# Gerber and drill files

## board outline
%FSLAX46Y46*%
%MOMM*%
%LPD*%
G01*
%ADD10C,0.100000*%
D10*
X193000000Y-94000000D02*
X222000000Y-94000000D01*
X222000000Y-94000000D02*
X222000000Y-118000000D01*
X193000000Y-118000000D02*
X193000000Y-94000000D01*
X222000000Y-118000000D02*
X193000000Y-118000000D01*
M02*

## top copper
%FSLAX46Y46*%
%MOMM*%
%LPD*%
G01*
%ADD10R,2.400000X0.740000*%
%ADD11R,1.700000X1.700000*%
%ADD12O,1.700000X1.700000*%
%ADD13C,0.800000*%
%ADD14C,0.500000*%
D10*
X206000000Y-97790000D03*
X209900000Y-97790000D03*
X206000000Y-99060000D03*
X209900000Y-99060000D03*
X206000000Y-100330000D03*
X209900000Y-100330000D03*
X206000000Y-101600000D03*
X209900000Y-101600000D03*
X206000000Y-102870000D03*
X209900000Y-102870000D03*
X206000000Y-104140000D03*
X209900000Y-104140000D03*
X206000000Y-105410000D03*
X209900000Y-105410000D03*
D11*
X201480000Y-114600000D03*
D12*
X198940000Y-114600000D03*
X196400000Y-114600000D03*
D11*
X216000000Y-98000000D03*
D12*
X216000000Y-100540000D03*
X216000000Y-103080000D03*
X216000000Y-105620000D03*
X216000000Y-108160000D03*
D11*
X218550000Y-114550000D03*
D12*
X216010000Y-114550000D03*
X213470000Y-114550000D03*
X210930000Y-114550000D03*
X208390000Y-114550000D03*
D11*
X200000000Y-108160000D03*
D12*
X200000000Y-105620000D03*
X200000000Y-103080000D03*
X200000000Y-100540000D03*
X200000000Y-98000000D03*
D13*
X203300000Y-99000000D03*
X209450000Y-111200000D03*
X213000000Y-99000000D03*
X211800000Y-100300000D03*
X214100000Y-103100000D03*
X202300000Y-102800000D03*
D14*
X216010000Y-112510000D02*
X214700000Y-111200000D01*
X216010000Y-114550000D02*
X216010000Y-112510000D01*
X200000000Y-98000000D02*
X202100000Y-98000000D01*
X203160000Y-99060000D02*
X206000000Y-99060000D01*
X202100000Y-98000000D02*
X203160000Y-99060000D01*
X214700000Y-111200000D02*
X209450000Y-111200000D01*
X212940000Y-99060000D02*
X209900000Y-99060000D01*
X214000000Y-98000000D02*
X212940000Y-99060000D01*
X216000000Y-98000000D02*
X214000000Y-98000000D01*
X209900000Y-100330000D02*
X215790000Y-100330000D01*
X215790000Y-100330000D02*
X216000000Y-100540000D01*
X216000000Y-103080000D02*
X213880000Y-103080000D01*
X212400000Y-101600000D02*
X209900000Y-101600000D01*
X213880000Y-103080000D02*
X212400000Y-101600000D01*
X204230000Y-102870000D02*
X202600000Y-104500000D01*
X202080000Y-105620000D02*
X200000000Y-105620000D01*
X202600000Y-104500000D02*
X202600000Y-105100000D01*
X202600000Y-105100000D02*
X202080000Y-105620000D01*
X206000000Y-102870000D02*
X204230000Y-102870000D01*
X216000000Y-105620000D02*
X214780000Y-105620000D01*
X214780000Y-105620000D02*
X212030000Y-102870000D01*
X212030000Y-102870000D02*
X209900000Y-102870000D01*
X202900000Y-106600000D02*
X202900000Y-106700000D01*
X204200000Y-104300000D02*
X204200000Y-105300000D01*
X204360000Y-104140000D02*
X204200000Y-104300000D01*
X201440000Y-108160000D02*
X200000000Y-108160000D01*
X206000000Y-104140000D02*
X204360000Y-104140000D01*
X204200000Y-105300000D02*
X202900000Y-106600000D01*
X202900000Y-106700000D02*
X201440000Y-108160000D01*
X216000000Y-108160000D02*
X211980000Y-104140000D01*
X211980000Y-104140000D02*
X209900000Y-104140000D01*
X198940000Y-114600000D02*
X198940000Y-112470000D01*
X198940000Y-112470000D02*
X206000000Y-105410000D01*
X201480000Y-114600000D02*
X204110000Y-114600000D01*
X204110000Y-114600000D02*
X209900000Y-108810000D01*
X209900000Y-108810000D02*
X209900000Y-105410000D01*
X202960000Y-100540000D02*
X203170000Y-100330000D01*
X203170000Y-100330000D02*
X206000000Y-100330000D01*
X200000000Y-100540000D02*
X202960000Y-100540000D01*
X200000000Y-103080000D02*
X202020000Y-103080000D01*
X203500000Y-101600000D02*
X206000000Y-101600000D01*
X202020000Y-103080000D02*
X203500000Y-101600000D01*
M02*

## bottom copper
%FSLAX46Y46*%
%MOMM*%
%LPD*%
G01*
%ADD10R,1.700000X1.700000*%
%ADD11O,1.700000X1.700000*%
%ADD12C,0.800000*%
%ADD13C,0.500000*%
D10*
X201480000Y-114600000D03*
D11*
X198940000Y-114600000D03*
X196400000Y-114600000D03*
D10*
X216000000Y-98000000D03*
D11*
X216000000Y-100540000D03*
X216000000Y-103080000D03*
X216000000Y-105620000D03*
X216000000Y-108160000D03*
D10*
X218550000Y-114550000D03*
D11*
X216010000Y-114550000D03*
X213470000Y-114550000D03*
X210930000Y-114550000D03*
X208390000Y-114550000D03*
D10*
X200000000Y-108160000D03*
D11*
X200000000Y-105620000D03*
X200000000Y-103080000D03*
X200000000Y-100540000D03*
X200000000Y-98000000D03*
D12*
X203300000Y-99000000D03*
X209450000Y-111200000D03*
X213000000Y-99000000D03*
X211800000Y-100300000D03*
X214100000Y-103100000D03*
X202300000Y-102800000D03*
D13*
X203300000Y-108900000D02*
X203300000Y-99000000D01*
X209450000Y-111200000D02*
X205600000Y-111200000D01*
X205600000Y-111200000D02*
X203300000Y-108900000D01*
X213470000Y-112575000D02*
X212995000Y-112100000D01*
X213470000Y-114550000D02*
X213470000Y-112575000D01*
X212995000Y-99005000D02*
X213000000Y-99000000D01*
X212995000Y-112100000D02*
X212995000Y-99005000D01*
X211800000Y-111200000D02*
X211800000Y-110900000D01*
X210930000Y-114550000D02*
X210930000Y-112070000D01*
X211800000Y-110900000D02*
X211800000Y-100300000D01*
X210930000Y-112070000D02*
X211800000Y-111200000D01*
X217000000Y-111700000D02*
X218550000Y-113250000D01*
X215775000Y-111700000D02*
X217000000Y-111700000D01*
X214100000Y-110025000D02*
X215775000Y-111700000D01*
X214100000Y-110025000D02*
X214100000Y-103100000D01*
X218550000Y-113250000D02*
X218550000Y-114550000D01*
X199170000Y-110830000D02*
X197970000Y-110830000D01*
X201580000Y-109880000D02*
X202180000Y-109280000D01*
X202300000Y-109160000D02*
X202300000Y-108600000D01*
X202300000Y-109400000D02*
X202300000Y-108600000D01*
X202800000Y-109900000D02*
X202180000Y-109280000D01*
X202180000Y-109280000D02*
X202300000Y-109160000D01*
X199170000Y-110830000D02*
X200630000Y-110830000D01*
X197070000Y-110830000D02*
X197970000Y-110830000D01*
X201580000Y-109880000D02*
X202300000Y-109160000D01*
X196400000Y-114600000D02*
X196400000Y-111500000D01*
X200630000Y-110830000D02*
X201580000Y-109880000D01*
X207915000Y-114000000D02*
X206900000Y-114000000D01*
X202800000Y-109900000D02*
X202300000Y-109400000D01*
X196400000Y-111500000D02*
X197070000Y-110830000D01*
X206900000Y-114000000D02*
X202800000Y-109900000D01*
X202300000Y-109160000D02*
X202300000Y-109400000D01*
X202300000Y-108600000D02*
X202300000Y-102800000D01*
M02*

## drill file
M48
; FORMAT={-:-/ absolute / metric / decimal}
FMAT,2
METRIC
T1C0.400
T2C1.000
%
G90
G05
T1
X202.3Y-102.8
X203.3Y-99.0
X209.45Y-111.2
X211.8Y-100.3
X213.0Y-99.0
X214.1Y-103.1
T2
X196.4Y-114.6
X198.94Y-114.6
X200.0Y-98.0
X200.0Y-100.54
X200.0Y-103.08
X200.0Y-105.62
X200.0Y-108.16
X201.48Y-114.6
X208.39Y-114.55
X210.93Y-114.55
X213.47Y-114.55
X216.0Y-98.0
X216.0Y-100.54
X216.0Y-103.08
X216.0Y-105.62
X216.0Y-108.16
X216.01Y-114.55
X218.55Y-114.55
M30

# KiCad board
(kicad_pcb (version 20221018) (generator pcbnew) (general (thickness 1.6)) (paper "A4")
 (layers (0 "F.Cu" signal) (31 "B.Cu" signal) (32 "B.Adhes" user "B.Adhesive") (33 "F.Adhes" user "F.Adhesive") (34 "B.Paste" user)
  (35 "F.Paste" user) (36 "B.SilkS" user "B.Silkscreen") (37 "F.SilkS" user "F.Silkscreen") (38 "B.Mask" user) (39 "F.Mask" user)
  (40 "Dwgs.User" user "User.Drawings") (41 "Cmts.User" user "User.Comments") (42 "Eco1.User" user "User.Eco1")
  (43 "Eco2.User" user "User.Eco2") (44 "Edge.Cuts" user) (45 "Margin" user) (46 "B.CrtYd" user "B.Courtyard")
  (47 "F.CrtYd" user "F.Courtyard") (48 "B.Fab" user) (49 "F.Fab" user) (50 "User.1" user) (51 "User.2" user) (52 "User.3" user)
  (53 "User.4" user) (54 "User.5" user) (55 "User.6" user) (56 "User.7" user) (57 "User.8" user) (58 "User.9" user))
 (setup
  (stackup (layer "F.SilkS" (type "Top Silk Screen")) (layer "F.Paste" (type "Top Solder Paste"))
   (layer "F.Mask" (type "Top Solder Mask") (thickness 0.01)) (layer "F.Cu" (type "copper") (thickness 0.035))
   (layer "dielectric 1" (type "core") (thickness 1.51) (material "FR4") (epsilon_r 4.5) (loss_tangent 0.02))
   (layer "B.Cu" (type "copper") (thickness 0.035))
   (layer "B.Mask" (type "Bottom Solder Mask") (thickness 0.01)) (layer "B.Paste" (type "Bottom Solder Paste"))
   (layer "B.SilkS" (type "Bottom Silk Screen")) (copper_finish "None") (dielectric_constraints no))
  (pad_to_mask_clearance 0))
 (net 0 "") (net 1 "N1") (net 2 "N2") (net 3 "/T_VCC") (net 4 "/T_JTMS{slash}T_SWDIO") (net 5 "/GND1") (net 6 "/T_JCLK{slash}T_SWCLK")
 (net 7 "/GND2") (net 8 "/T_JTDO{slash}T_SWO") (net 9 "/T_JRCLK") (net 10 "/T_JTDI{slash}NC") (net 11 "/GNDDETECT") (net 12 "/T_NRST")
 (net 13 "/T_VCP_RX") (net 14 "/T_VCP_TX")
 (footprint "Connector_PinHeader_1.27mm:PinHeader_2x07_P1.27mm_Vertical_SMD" (layer "F.Cu") (at 207.95 101.6)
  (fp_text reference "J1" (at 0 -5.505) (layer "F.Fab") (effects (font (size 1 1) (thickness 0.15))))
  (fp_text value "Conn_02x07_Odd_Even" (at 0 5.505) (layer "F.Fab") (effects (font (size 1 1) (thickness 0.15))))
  (pad "1" smd rect (at -1.95 -3.81) (size 2.4 0.74) (layers "F.Cu" "F.Paste" "F.Mask") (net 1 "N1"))
  (pad "2" smd rect (at 1.95 -3.81) (size 2.4 0.74) (layers "F.Cu" "F.Paste" "F.Mask") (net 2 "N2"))
  (pad "3" smd rect (at -1.95 -2.54) (size 2.4 0.74) (layers "F.Cu" "F.Paste" "F.Mask") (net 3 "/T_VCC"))
  (pad "4" smd rect (at 1.95 -2.54) (size 2.4 0.74) (layers "F.Cu" "F.Paste" "F.Mask") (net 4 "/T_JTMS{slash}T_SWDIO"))
  (pad "5" smd rect (at -1.95 -1.27) (size 2.4 0.74) (layers "F.Cu" "F.Paste" "F.Mask") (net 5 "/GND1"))
  (pad "6" smd rect (at 1.95 -1.27) (size 2.4 0.74) (layers "F.Cu" "F.Paste" "F.Mask") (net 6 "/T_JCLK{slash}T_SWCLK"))
  (pad "7" smd rect (at -1.95 0) (size 2.4 0.74) (layers "F.Cu" "F.Paste" "F.Mask") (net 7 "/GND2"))
  (pad "8" smd rect (at 1.95 0) (size 2.4 0.74) (layers "F.Cu" "F.Paste" "F.Mask") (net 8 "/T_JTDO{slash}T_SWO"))
  (pad "9" smd rect (at -1.95 1.27) (size 2.4 0.74) (layers "F.Cu" "F.Paste" "F.Mask") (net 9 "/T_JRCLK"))
  (pad "10" smd rect (at 1.95 1.27) (size 2.4 0.74) (layers "F.Cu" "F.Paste" "F.Mask") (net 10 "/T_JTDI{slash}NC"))
  (pad "11" smd rect (at -1.95 2.54) (size 2.4 0.74) (layers "F.Cu" "F.Paste" "F.Mask") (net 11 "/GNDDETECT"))
  (pad "12" smd rect (at 1.95 2.54) (size 2.4 0.74) (layers "F.Cu" "F.Paste" "F.Mask") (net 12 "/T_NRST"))
  (pad "13" smd rect (at -1.95 3.81) (size 2.4 0.74) (layers "F.Cu" "F.Paste" "F.Mask") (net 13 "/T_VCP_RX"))
  (pad "14" smd rect (at 1.95 3.81) (size 2.4 0.74) (layers "F.Cu" "F.Paste" "F.Mask") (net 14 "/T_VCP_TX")))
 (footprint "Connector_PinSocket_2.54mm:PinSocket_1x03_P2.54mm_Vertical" (layer "B.Cu") (at 201.48 114.6 90)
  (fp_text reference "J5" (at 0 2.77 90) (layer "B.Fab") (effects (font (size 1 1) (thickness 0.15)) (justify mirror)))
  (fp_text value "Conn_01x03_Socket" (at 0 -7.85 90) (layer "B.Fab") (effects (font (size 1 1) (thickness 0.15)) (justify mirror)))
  (pad "1" thru_hole rect (at 0 0 90) (size 1.7 1.7) (drill 1) (layers "*.Cu" "*.Mask") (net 14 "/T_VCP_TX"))
  (pad "2" thru_hole oval (at 0 -2.54 90) (size 1.7 1.7) (drill 1) (layers "*.Cu" "*.Mask") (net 13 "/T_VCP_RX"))
  (pad "3" thru_hole oval (at 0 -5.08 90) (size 1.7 1.7) (drill 1) (layers "*.Cu" "*.Mask") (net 7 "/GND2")))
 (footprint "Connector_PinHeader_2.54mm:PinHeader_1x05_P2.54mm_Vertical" (layer "B.Cu") (at 216 98 180)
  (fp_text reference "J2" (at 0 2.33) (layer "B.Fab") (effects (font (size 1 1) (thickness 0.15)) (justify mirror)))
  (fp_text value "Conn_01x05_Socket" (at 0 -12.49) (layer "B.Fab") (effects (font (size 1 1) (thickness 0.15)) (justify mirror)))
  (pad "1" thru_hole rect (at 0 0 180) (size 1.7 1.7) (drill 1) (layers "*.Cu" "*.Mask") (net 4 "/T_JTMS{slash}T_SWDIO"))
  (pad "2" thru_hole oval (at 0 -2.54 180) (size 1.7 1.7) (drill 1) (layers "*.Cu" "*.Mask") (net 6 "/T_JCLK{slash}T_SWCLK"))
  (pad "3" thru_hole oval (at 0 -5.08 180) (size 1.7 1.7) (drill 1) (layers "*.Cu" "*.Mask") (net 8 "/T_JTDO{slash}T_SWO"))
  (pad "4" thru_hole oval (at 0 -7.62 180) (size 1.7 1.7) (drill 1) (layers "*.Cu" "*.Mask") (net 10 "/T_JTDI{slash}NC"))
  (pad "5" thru_hole oval (at 0 -10.16 180) (size 1.7 1.7) (drill 1) (layers "*.Cu" "*.Mask") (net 12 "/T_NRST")))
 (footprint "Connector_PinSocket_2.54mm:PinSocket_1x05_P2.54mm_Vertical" (layer "B.Cu") (at 218.55 114.55 90)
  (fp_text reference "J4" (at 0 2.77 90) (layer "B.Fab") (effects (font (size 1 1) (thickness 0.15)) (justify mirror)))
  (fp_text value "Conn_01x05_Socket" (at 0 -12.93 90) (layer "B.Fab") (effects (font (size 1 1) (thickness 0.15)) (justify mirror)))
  (pad "1" thru_hole rect (at 0 0 90) (size 1.7 1.7) (drill 1) (layers "*.Cu" "*.Mask") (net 8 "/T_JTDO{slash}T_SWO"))
  (pad "2" thru_hole oval (at 0 -2.54 90) (size 1.7 1.7) (drill 1) (layers "*.Cu" "*.Mask") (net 3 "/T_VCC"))
  (pad "3" thru_hole oval (at 0 -5.08 90) (size 1.7 1.7) (drill 1) (layers "*.Cu" "*.Mask") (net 4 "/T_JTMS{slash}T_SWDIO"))
  (pad "4" thru_hole oval (at 0 -7.62 90) (size 1.7 1.7) (drill 1) (layers "*.Cu" "*.Mask") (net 6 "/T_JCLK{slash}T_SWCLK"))
  (pad "5" thru_hole oval (at 0 -10.16 90) (size 1.7 1.7) (drill 1) (layers "*.Cu" "*.Mask") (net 7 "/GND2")))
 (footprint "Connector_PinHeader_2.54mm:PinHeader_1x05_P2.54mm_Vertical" (layer "B.Cu") (at 200 108.16)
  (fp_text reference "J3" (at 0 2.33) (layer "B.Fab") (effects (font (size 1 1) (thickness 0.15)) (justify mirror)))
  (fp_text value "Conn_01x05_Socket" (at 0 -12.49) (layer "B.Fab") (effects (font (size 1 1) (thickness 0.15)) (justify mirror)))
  (pad "1" thru_hole rect (at 0 0) (size 1.7 1.7) (drill 1) (layers "*.Cu" "*.Mask") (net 11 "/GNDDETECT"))
  (pad "2" thru_hole oval (at 0 -2.54) (size 1.7 1.7) (drill 1) (layers "*.Cu" "*.Mask") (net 9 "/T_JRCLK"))
  (pad "3" thru_hole oval (at 0 -5.08) (size 1.7 1.7) (drill 1) (layers "*.Cu" "*.Mask") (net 7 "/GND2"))
  (pad "4" thru_hole oval (at 0 -7.62) (size 1.7 1.7) (drill 1) (layers "*.Cu" "*.Mask") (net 5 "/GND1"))
  (pad "5" thru_hole oval (at 0 -10.16) (size 1.7 1.7) (drill 1) (layers "*.Cu" "*.Mask") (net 3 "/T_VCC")))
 (gr_line (start 193 94) (end 222 94) (stroke (width 0.1) (type default)) (layer "Edge.Cuts"))
 (gr_line (start 222 94) (end 222 118) (stroke (width 0.1) (type default)) (layer "Edge.Cuts"))
 (gr_line (start 193 118) (end 193 94) (stroke (width 0.1) (type default)) (layer "Edge.Cuts"))
 (gr_line (start 222 118) (end 193 118) (stroke (width 0.1) (type default)) (layer "Edge.Cuts"))
 (segment (start 216.01 112.51) (end 214.7 111.2) (width 0.5) (layer "F.Cu") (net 3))
 (segment (start 216.01 114.55) (end 216.01 112.51) (width 0.5) (layer "F.Cu") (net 3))
 (segment (start 200 98) (end 202.1 98) (width 0.5) (layer "F.Cu") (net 3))
 (segment (start 203.16 99.06) (end 206 99.06) (width 0.5) (layer "F.Cu") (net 3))
 (segment (start 202.1 98) (end 203.16 99.06) (width 0.5) (layer "F.Cu") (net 3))
 (segment (start 214.7 111.2) (end 209.45 111.2) (width 0.5) (layer "F.Cu") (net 3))
 (via (at 203.3 99) (size 0.8) (drill 0.4) (layers "F.Cu" "B.Cu") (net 3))
 (via (at 209.45 111.2) (size 0.8) (drill 0.4) (layers "F.Cu" "B.Cu") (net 3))
 (segment (start 203.3 108.9) (end 203.3 99) (width 0.5) (layer "B.Cu") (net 3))
 (segment (start 209.45 111.2) (end 205.6 111.2) (width 0.5) (layer "B.Cu") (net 3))
 (segment (start 205.6 111.2) (end 203.3 108.9) (width 0.5) (layer "B.Cu") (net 3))
 (segment (start 212.94 99.06) (end 209.9 99.06) (width 0.5) (layer "F.Cu") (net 4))
 (segment (start 214 98) (end 212.94 99.06) (width 0.5) (layer "F.Cu") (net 4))
 (segment (start 216 98) (end 214 98) (width 0.5) (layer "F.Cu") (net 4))
 (via (at 213 99) (size 0.8) (drill 0.4) (layers "F.Cu" "B.Cu") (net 4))
 (segment (start 213.47 112.575) (end 212.995 112.1) (width 0.5) (layer "B.Cu") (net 4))
 (segment (start 213.47 114.55) (end 213.47 112.575) (width 0.5) (layer "B.Cu") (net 4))
 (segment (start 212.995 99.005) (end 213 99) (width 0.5) (layer "B.Cu") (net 4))
 (segment (start 212.995 112.1) (end 212.995 99.005) (width 0.5) (layer "B.Cu") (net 4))
 (segment (start 209.9 100.33) (end 215.79 100.33) (width 0.5) (layer "F.Cu") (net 6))
 (segment (start 215.79 100.33) (end 216 100.54) (width 0.5) (layer "F.Cu") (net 6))
 (via (at 211.8 100.3) (size 0.8) (drill 0.4) (layers "F.Cu" "B.Cu") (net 6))
 (segment (start 211.8 111.2) (end 211.8 110.9) (width 0.5) (layer "B.Cu") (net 6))
 (segment (start 210.93 114.55) (end 210.93 112.07) (width 0.5) (layer "B.Cu") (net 6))
 (segment (start 211.8 110.9) (end 211.8 100.3) (width 0.5) (layer "B.Cu") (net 6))
 (segment (start 210.93 112.07) (end 211.8 111.2) (width 0.5) (layer "B.Cu") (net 6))
 (segment (start 216 103.08) (end 213.88 103.08) (width 0.5) (layer "F.Cu") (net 8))
 (segment (start 212.4 101.6) (end 209.9 101.6) (width 0.5) (layer "F.Cu") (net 8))
 (segment (start 213.88 103.08) (end 212.4 101.6) (width 0.5) (layer "F.Cu") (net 8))
 (via (at 214.1 103.1) (size 0.8) (drill 0.4) (layers "F.Cu" "B.Cu") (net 8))
 (segment (start 217 111.7) (end 218.55 113.25) (width 0.5) (layer "B.Cu") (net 8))
 (segment (start 215.775 111.7) (end 217 111.7) (width 0.5) (layer "B.Cu") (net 8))
 (segment (start 214.1 110.025) (end 215.775 111.7) (width 0.5) (layer "B.Cu") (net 8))
 (segment (start 214.1 110.025) (end 214.1 103.1) (width 0.5) (layer "B.Cu") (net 8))
 (segment (start 218.55 113.25) (end 218.55 114.55) (width 0.5) (layer "B.Cu") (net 8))
 (segment (start 204.23 102.87) (end 202.6 104.5) (width 0.5) (layer "F.Cu") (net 9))
 (segment (start 202.08 105.62) (end 200 105.62) (width 0.5) (layer "F.Cu") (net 9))
 (segment (start 202.6 104.5) (end 202.6 105.1) (width 0.5) (layer "F.Cu") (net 9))
 (segment (start 202.6 105.1) (end 202.08 105.62) (width 0.5) (layer "F.Cu") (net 9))
 (segment (start 206 102.87) (end 204.23 102.87) (width 0.5) (layer "F.Cu") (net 9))
 (segment (start 216 105.62) (end 214.78 105.62) (width 0.5) (layer "F.Cu") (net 10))
 (segment (start 214.78 105.62) (end 212.03 102.87) (width 0.5) (layer "F.Cu") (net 10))
 (segment (start 212.03 102.87) (end 209.9 102.87) (width 0.5) (layer "F.Cu") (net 10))
 (segment (start 202.9 106.6) (end 202.9 106.7) (width 0.5) (layer "F.Cu") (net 11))
 (segment (start 204.2 104.3) (end 204.2 105.3) (width 0.5) (layer "F.Cu") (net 11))
 (segment (start 204.36 104.14) (end 204.2 104.3) (width 0.5) (layer "F.Cu") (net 11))
 (segment (start 201.44 108.16) (end 200 108.16) (width 0.5) (layer "F.Cu") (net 11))
 (segment (start 206 104.14) (end 204.36 104.14) (width 0.5) (layer "F.Cu") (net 11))
 (segment (start 204.2 105.3) (end 202.9 106.6) (width 0.5) (layer "F.Cu") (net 11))
 (segment (start 202.9 106.7) (end 201.44 108.16) (width 0.5) (layer "F.Cu") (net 11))
 (segment (start 216 108.16) (end 211.98 104.14) (width 0.5) (layer "F.Cu") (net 12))
 (segment (start 211.98 104.14) (end 209.9 104.14) (width 0.5) (layer "F.Cu") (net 12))
 (segment (start 198.94 114.6) (end 198.94 112.47) (width 0.5) (layer "F.Cu") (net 13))
 (segment (start 198.94 112.47) (end 206 105.41) (width 0.5) (layer "F.Cu") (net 13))
 (segment (start 201.48 114.6) (end 204.11 114.6) (width 0.5) (layer "F.Cu") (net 14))
 (segment (start 204.11 114.6) (end 209.9 108.81) (width 0.5) (layer "F.Cu") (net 14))
 (segment (start 209.9 108.81) (end 209.9 105.41) (width 0.5) (layer "F.Cu") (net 14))
 (segment (start 202.96 100.54) (end 203.17 100.33) (width 0.5) (layer "F.Cu") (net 5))
 (segment (start 203.17 100.33) (end 206 100.33) (width 0.5) (layer "F.Cu") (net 5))
 (segment (start 200 100.54) (end 202.96 100.54) (width 0.5) (layer "F.Cu") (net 5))
 (segment (start 200 103.08) (end 202.02 103.08) (width 0.5) (layer "F.Cu") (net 7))
 (segment (start 203.5 101.6) (end 206 101.6) (width 0.5) (layer "F.Cu") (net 7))
 (segment (start 202.02 103.08) (end 203.5 101.6) (width 0.5) (layer "F.Cu") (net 7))
 (via (at 202.3 102.8) (size 0.8) (drill 0.4) (layers "F.Cu" "B.Cu") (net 7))
 (segment (start 199.17 110.83) (end 197.97 110.83) (width 0.5) (layer "B.Cu") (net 7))
 (segment (start 201.58 109.88) (end 202.18 109.28) (width 0.5) (layer "B.Cu") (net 7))
 (segment (start 202.3 109.16) (end 202.3 108.6) (width 0.5) (layer "B.Cu") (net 7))
 (segment (start 202.3 109.4) (end 202.3 108.6) (width 0.5) (layer "B.Cu") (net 7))
 (segment (start 202.8 109.9) (end 202.18 109.28) (width 0.5) (layer "B.Cu") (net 7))
 (segment (start 202.18 109.28) (end 202.3 109.16) (width 0.5) (layer "B.Cu") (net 7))
 (segment (start 199.17 110.83) (end 200.63 110.83) (width 0.5) (layer "B.Cu") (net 7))
 (segment (start 197.07 110.83) (end 197.97 110.83) (width 0.5) (layer "B.Cu") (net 7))
 (segment (start 201.58 109.88) (end 202.3 109.16) (width 0.5) (layer "B.Cu") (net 7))
 (segment (start 196.4 114.6) (end 196.4 111.5) (width 0.5) (layer "B.Cu") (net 7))
 (segment (start 200.63 110.83) (end 201.58 109.88) (width 0.5) (layer "B.Cu") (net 7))
 (segment (start 207.915 114) (end 206.9 114) (width 0.5) (layer "B.Cu") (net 7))
 (segment (start 202.8 109.9) (end 202.3 109.4) (width 0.5) (layer "B.Cu") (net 7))
 (segment (start 196.4 111.5) (end 197.07 110.83) (width 0.5) (layer "B.Cu") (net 7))
 (segment (start 206.9 114) (end 202.8 109.9) (width 0.5) (layer "B.Cu") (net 7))
 (segment (start 202.3 109.16) (end 202.3 109.4) (width 0.5) (layer "B.Cu") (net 7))
 (segment (start 202.3 108.6) (end 202.3 102.8) (width 0.5) (layer "B.Cu") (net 7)))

